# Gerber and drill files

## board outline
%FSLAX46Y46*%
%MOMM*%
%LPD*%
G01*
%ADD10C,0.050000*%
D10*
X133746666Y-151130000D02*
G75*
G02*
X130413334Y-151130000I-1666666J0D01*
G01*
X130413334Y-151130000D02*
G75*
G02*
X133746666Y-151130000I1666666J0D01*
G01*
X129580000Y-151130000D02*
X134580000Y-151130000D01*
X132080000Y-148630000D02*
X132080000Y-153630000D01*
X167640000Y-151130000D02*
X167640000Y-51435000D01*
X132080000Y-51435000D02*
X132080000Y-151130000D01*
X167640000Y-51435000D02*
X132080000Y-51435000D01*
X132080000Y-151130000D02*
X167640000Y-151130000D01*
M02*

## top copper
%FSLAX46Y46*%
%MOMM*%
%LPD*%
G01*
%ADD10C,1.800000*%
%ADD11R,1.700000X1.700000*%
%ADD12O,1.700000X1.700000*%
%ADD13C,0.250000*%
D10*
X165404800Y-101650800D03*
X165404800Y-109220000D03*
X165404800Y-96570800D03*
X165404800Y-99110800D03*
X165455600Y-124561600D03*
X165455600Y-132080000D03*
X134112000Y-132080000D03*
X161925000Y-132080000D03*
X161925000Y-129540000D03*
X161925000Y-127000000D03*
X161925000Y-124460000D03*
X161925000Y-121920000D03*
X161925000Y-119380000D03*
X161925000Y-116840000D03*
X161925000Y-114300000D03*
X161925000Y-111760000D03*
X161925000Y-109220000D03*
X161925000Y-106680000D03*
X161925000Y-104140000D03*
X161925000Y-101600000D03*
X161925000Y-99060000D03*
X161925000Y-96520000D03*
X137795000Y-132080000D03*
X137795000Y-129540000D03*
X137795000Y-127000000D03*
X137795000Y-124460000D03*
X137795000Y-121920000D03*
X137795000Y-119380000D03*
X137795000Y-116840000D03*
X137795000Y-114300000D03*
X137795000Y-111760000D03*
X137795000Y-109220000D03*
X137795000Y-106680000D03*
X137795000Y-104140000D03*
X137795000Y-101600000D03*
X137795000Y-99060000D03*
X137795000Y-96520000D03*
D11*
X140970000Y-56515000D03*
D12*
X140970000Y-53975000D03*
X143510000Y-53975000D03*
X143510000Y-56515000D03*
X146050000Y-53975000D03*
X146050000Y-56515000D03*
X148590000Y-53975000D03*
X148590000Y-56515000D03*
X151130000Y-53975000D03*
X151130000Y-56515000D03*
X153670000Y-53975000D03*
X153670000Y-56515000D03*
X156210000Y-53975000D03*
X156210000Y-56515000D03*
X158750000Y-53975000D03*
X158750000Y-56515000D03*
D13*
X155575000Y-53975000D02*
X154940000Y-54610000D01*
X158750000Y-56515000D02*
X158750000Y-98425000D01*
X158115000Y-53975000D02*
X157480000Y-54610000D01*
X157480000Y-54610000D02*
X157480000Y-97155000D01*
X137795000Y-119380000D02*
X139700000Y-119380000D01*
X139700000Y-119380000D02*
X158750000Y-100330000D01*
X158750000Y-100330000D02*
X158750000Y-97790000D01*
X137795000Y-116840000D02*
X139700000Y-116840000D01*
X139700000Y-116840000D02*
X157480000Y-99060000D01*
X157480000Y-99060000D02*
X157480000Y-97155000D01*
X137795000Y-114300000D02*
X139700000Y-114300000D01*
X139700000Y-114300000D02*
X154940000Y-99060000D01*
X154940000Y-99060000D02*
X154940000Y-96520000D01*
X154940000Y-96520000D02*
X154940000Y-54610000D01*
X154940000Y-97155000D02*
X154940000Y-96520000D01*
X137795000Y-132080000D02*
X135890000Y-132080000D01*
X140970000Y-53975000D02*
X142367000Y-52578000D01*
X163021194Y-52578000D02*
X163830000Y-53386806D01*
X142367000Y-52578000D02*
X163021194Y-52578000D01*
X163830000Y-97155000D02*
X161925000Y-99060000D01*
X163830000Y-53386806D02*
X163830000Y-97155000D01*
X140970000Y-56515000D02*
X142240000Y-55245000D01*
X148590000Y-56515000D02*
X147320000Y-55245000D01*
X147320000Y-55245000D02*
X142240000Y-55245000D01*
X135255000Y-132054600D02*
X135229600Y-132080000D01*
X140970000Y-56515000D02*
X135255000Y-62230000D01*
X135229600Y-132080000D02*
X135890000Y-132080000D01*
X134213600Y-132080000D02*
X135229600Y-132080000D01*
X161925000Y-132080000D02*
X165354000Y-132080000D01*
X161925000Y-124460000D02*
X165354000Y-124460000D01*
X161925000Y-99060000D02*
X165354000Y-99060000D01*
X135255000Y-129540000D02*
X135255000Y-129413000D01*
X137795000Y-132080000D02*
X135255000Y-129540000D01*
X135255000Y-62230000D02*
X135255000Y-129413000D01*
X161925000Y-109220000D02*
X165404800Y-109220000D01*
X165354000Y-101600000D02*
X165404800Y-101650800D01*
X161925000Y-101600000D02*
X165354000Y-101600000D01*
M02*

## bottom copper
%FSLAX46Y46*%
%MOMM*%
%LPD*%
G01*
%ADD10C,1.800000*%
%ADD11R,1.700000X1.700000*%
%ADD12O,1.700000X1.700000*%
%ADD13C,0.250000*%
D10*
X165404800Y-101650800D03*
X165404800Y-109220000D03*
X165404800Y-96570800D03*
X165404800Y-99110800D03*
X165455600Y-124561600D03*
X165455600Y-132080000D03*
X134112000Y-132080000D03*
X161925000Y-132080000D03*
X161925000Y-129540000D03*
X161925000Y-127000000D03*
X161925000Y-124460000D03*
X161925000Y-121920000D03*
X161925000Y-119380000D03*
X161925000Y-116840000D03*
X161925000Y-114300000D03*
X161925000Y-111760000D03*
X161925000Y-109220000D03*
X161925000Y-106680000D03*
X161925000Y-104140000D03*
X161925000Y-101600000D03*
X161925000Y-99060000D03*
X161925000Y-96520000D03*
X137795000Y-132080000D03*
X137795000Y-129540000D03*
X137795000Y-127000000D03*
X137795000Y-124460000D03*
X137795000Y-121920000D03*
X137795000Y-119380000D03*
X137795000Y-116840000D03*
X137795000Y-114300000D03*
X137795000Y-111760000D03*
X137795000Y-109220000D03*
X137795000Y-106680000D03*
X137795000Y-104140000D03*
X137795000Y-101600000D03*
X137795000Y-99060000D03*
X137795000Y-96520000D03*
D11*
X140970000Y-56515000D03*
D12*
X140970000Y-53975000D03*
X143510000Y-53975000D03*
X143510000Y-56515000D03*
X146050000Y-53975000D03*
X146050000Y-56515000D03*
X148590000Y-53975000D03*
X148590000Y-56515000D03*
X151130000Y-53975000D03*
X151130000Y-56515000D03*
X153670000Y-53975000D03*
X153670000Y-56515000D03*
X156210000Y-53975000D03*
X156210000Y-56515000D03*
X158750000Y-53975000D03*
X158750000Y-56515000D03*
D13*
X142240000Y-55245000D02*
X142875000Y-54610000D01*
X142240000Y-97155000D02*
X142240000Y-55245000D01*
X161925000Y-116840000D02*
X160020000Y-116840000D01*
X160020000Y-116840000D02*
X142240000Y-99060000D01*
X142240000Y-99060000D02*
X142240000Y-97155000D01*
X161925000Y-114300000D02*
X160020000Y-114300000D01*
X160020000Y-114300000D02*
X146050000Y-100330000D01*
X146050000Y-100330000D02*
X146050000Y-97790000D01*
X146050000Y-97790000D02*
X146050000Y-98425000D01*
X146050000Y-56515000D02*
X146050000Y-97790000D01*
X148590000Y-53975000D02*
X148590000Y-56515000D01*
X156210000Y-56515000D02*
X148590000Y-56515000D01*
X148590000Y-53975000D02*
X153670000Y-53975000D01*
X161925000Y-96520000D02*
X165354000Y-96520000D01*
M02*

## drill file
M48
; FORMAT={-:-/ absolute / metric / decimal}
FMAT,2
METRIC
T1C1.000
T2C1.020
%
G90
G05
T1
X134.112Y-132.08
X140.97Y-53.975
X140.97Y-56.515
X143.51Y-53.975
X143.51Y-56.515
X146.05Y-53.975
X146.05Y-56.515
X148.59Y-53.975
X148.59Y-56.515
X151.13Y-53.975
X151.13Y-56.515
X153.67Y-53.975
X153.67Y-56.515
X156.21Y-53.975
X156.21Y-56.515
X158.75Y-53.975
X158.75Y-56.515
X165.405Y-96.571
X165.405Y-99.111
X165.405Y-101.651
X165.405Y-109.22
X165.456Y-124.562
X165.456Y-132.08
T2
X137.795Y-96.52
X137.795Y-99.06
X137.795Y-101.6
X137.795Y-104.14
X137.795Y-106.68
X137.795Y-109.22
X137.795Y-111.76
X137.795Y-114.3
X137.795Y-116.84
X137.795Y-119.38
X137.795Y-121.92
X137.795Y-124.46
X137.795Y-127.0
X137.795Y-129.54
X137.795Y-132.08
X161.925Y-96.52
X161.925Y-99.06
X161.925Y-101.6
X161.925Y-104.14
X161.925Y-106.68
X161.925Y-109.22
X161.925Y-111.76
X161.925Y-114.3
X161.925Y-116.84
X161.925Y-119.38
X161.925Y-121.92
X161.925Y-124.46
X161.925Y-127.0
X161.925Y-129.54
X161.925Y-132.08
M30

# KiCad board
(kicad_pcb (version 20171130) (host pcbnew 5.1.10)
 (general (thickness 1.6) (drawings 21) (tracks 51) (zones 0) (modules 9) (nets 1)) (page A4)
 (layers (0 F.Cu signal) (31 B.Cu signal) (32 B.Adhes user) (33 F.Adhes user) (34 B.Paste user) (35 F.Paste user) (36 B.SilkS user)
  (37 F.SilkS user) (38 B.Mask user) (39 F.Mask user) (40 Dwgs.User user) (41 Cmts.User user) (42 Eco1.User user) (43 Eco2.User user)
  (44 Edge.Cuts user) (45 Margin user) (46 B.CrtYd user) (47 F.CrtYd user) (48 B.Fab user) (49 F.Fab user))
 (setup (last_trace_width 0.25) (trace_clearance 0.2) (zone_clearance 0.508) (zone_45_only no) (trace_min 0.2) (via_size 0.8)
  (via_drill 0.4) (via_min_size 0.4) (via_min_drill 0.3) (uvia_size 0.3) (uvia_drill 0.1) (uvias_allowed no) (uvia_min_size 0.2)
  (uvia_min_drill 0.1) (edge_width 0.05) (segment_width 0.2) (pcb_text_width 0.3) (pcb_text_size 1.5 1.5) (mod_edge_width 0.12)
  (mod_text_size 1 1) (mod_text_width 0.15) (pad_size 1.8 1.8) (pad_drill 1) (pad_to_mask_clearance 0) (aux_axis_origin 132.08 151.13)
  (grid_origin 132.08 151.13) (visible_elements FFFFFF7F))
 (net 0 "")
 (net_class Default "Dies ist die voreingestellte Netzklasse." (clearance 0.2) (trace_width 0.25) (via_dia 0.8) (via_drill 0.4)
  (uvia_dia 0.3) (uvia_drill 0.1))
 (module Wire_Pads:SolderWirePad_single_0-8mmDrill (layer F.Cu) (at 165.4048 101.6508)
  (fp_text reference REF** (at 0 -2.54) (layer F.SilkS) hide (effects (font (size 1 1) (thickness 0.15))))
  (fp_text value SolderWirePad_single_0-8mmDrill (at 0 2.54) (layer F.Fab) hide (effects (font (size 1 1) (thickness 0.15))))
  (pad 1 thru_hole circle (at 0 0) (size 1.8 1.8) (drill 1) (layers *.Cu *.Mask)))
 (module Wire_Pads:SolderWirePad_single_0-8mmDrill (layer F.Cu) (at 165.4048 109.22)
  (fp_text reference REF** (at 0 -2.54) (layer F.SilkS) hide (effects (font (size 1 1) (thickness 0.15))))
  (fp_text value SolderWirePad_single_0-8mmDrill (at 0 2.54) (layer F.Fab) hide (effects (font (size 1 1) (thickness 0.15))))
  (pad 1 thru_hole circle (at 0 0) (size 1.8 1.8) (drill 1) (layers *.Cu *.Mask)))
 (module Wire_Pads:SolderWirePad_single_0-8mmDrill (layer F.Cu) (at 165.4048 96.5708)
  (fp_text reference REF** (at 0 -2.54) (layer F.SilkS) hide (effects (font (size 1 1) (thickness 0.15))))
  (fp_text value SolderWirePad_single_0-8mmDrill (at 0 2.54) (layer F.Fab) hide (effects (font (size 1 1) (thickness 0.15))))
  (pad 1 thru_hole circle (at 0 0) (size 1.8 1.8) (drill 1) (layers *.Cu *.Mask)))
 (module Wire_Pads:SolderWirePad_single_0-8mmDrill (layer F.Cu) (at 165.4048 99.1108)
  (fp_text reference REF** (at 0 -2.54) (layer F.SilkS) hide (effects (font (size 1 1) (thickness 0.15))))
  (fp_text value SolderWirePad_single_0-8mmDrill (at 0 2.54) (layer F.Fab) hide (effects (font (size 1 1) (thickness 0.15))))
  (pad 1 thru_hole circle (at 0 0) (size 1.8 1.8) (drill 1) (layers *.Cu *.Mask)))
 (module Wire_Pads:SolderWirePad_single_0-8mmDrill (layer F.Cu) (at 165.4556 124.5616)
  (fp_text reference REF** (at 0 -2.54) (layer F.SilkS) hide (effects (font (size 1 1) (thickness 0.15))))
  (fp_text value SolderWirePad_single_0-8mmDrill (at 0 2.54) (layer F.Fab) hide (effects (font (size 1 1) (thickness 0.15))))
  (pad 1 thru_hole circle (at 0 0) (size 1.8 1.8) (drill 1) (layers *.Cu *.Mask)))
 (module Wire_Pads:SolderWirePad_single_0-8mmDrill (layer F.Cu) (at 165.4556 132.08)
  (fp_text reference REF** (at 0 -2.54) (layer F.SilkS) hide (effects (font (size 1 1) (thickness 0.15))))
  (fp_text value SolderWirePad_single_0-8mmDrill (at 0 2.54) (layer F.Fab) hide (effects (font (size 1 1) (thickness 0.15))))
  (pad 1 thru_hole circle (at 0 0) (size 1.8 1.8) (drill 1) (layers *.Cu *.Mask)))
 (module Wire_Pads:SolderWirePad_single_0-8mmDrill (layer F.Cu) (at 134.112 132.08)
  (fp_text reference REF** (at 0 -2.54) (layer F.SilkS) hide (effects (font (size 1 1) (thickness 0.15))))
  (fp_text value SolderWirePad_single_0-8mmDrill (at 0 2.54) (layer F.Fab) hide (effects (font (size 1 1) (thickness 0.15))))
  (pad 1 thru_hole circle (at 0 0) (size 1.8 1.8) (drill 1) (layers *.Cu *.Mask)))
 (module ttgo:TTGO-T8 (layer F.Cu) (at 137.795 96.52)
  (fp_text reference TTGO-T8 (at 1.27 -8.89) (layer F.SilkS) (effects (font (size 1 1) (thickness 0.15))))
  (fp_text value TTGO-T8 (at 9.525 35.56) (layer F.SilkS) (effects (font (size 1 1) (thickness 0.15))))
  (pad 5V thru_hole circle (at 24.13 35.56) (size 1.8 1.8) (drill 1.02) (layers *.Cu *.Mask))
  (pad 4 thru_hole circle (at 24.13 33.02) (size 1.8 1.8) (drill 1.02) (layers *.Cu *.Mask))
  (pad 0 thru_hole circle (at 24.13 30.48) (size 1.8 1.8) (drill 1.02) (layers *.Cu *.Mask))
  (pad GND thru_hole circle (at 24.13 27.94) (size 1.8 1.8) (drill 1.02) (layers *.Cu *.Mask))
  (pad 2 thru_hole circle (at 24.13 25.4) (size 1.8 1.8) (drill 1.02) (layers *.Cu *.Mask))
  (pad 5 thru_hole circle (at 24.13 22.86) (size 1.8 1.8) (drill 1.02) (layers *.Cu *.Mask))
  (pad 18 thru_hole circle (at 24.13 20.32) (size 1.8 1.8) (drill 1.02) (layers *.Cu *.Mask))
  (pad 23 thru_hole circle (at 24.13 17.78) (size 1.8 1.8) (drill 1.02) (layers *.Cu *.Mask))
  (pad 19 thru_hole circle (at 24.13 15.24) (size 1.8 1.8) (drill 1.02) (layers *.Cu *.Mask))
  (pad 22 thru_hole circle (at 24.13 12.7) (size 1.8 1.8) (drill 1.02) (layers *.Cu *.Mask))
  (pad RXD thru_hole circle (at 24.13 10.16) (size 1.8 1.8) (drill 1.02) (layers *.Cu *.Mask))
  (pad TXD thru_hole circle (at 24.13 7.62) (size 1.8 1.8) (drill 1.02) (layers *.Cu *.Mask))
  (pad 21 thru_hole circle (at 24.13 5.08) (size 1.8 1.8) (drill 1.02) (layers *.Cu *.Mask))
  (pad 3-3 thru_hole circle (at 24.13 2.54) (size 1.8 1.8) (drill 1.02) (layers *.Cu *.Mask))
  (pad GND thru_hole circle (at 24.13 0) (size 1.8 1.8) (drill 1.02) (layers *.Cu *.Mask))
  (pad GND thru_hole circle (at 0 35.56) (size 1.8 1.8) (drill 1.02) (layers *.Cu *.Mask))
  (pad 15 thru_hole circle (at 0 33.02) (size 1.8 1.8) (drill 1.02) (layers *.Cu *.Mask))
  (pad 13 thru_hole circle (at 0 30.48) (size 1.8 1.8) (drill 1.02) (layers *.Cu *.Mask))
  (pad 12 thru_hole circle (at 0 27.94) (size 1.8 1.8) (drill 1.02) (layers *.Cu *.Mask))
  (pad 14 thru_hole circle (at 0 25.4) (size 1.8 1.8) (drill 1.02) (layers *.Cu *.Mask))
  (pad 27 thru_hole circle (at 0 22.86) (size 1.8 1.8) (drill 1.02) (layers *.Cu *.Mask))
  (pad 26 thru_hole circle (at 0 20.32) (size 1.8 1.8) (drill 1.02) (layers *.Cu *.Mask))
  (pad 25 thru_hole circle (at 0 17.78) (size 1.8 1.8) (drill 1.02) (layers *.Cu *.Mask))
  (pad 33 thru_hole circle (at 0 15.24) (size 1.8 1.8) (drill 1.02) (layers *.Cu *.Mask))
  (pad 32 thru_hole circle (at 0 12.7) (size 1.8 1.8) (drill 1.02) (layers *.Cu *.Mask))
  (pad 35 thru_hole circle (at 0 10.16) (size 1.8 1.8) (drill 1.02) (layers *.Cu *.Mask))
  (pad 34 thru_hole circle (at 0 7.62) (size 1.8 1.8) (drill 1.02) (layers *.Cu *.Mask))
  (pad RST thru_hole circle (at 0 5.08) (size 1.8 1.8) (drill 1.02) (layers *.Cu *.Mask))
  (pad VN thru_hole circle (at 0 2.54) (size 1.8 1.8) (drill 1.02) (layers *.Cu *.Mask))
  (pad VP thru_hole circle (at 0 0) (size 1.8 1.8) (drill 1.02) (layers *.Cu *.Mask)))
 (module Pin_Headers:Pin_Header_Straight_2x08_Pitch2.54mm (layer B.Cu) (at 140.97 53.975 270)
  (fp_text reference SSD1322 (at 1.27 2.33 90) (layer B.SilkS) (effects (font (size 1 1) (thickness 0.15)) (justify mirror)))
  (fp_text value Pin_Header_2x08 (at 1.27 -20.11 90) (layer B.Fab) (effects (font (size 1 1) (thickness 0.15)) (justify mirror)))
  (pad 1 thru_hole rect (at 2.54 0 270) (size 1.7 1.7) (drill 1) (layers *.Cu *.Mask))
  (pad 2 thru_hole oval (at 0 0 270) (size 1.7 1.7) (drill 1) (layers *.Cu *.Mask))
  (pad 4 thru_hole oval (at 0 -2.54 270) (size 1.7 1.7) (drill 1) (layers *.Cu *.Mask))
  (pad 3 thru_hole oval (at 2.54 -2.54 270) (size 1.7 1.7) (drill 1) (layers *.Cu *.Mask))
  (pad 6 thru_hole oval (at 0 -5.08 270) (size 1.7 1.7) (drill 1) (layers *.Cu *.Mask))
  (pad 5 thru_hole oval (at 2.54 -5.08 270) (size 1.7 1.7) (drill 1) (layers *.Cu *.Mask))
  (pad 8 thru_hole oval (at 0 -7.62 270) (size 1.7 1.7) (drill 1) (layers *.Cu *.Mask))
  (pad 7 thru_hole oval (at 2.54 -7.62 270) (size 1.7 1.7) (drill 1) (layers *.Cu *.Mask))
  (pad 10 thru_hole oval (at 0 -10.16 270) (size 1.7 1.7) (drill 1) (layers *.Cu *.Mask))
  (pad 9 thru_hole oval (at 2.54 -10.16 270) (size 1.7 1.7) (drill 1) (layers *.Cu *.Mask))
  (pad 12 thru_hole oval (at 0 -12.7 270) (size 1.7 1.7) (drill 1) (layers *.Cu *.Mask))
  (pad 11 thru_hole oval (at 2.54 -12.7 270) (size 1.7 1.7) (drill 1) (layers *.Cu *.Mask))
  (pad 14 thru_hole oval (at 0 -15.24 270) (size 1.7 1.7) (drill 1) (layers *.Cu *.Mask))
  (pad 13 thru_hole oval (at 2.54 -15.24 270) (size 1.7 1.7) (drill 1) (layers *.Cu *.Mask))
  (pad 16 thru_hole oval (at 0 -17.78 270) (size 1.7 1.7) (drill 1) (layers *.Cu *.Mask))
  (pad 15 thru_hole oval (at 2.54 -17.78 270) (size 1.7 1.7) (drill 1) (layers *.Cu *.Mask)))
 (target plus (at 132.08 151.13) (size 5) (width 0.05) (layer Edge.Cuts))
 (gr_line (start 167.64 151.13) (end 167.64 51.435) (layer Edge.Cuts) (width 0.05))
 (gr_line (start 132.08 51.435) (end 132.08 151.13) (layer Edge.Cuts) (width 0.05))
 (gr_line (start 167.64 51.435) (end 132.08 51.435) (layer Edge.Cuts) (width 0.05))
 (gr_line (start 132.08 151.13) (end 167.64 151.13) (layer Edge.Cuts) (width 0.05))
 (segment (start 142.24 55.245) (end 142.875 54.61) (width 0.25) (layer B.Cu) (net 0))
 (segment (start 142.24 97.155) (end 142.24 55.245) (width 0.25) (layer B.Cu) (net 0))
 (segment (start 155.575 53.975) (end 154.94 54.61) (width 0.25) (layer F.Cu) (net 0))
 (segment (start 158.75 56.515) (end 158.75 98.425) (width 0.25) (layer F.Cu) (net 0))
 (segment (start 158.115 53.975) (end 157.48 54.61) (width 0.25) (layer F.Cu) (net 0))
 (segment (start 157.48 54.61) (end 157.48 97.155) (width 0.25) (layer F.Cu) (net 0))
 (segment (start 161.925 116.84) (end 160.02 116.84) (width 0.25) (layer B.Cu) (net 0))
 (segment (start 160.02 116.84) (end 142.24 99.06) (width 0.25) (layer B.Cu) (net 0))
 (segment (start 142.24 99.06) (end 142.24 97.155) (width 0.25) (layer B.Cu) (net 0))
 (segment (start 161.925 114.3) (end 160.02 114.3) (width 0.25) (layer B.Cu) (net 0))
 (segment (start 160.02 114.3) (end 146.05 100.33) (width 0.25) (layer B.Cu) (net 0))
 (segment (start 146.05 100.33) (end 146.05 97.79) (width 0.25) (layer B.Cu) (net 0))
 (segment (start 146.05 97.79) (end 146.05 98.425) (width 0.25) (layer B.Cu) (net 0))
 (segment (start 146.05 56.515) (end 146.05 97.79) (width 0.25) (layer B.Cu) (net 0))
 (segment (start 137.795 119.38) (end 139.7 119.38) (width 0.25) (layer F.Cu) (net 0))
 (segment (start 139.7 119.38) (end 158.75 100.33) (width 0.25) (layer F.Cu) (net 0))
 (segment (start 158.75 100.33) (end 158.75 97.79) (width 0.25) (layer F.Cu) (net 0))
 (segment (start 137.795 116.84) (end 139.7 116.84) (width 0.25) (layer F.Cu) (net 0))
 (segment (start 139.7 116.84) (end 157.48 99.06) (width 0.25) (layer F.Cu) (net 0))
 (segment (start 157.48 99.06) (end 157.48 97.155) (width 0.25) (layer F.Cu) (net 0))
 (segment (start 137.795 114.3) (end 139.7 114.3) (width 0.25) (layer F.Cu) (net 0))
 (segment (start 139.7 114.3) (end 154.94 99.06) (width 0.25) (layer F.Cu) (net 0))
 (segment (start 154.94 99.06) (end 154.94 96.52) (width 0.25) (layer F.Cu) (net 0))
 (segment (start 154.94 96.52) (end 154.94 54.61) (width 0.25) (layer F.Cu) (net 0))
 (segment (start 154.94 97.155) (end 154.94 96.52) (width 0.25) (layer F.Cu) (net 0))
 (segment (start 137.795 132.08) (end 135.89 132.08) (width 0.25) (layer F.Cu) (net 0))
 (segment (start 140.97 53.975) (end 142.367 52.578) (width 0.25) (layer F.Cu) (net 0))
 (segment (start 163.021194 52.578) (end 163.83 53.386806) (width 0.25) (layer F.Cu) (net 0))
 (segment (start 142.367 52.578) (end 163.021194 52.578) (width 0.25) (layer F.Cu) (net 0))
 (segment (start 163.83 97.155) (end 161.925 99.06) (width 0.25) (layer F.Cu) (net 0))
 (segment (start 163.83 53.386806) (end 163.83 97.155) (width 0.25) (layer F.Cu) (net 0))
 (segment (start 148.59 53.975) (end 148.59 56.515) (width 0.25) (layer B.Cu) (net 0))
 (segment (start 156.21 56.515) (end 148.59 56.515) (width 0.25) (layer B.Cu) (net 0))
 (segment (start 148.59 53.975) (end 153.67 53.975) (width 0.25) (layer B.Cu) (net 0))
 (segment (start 140.97 56.515) (end 142.24 55.245) (width 0.25) (layer F.Cu) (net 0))
 (segment (start 148.59 56.515) (end 147.32 55.245) (width 0.25) (layer F.Cu) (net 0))
 (segment (start 147.32 55.245) (end 142.24 55.245) (width 0.25) (layer F.Cu) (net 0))
 (segment (start 135.255 132.0546) (end 135.2296 132.08) (width 0.25) (layer F.Cu) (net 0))
 (segment (start 140.97 56.515) (end 135.255 62.23) (width 0.25) (layer F.Cu) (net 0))
 (segment (start 135.2296 132.08) (end 135.89 132.08) (width 0.25) (layer F.Cu) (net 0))
 (segment (start 134.2136 132.08) (end 135.2296 132.08) (width 0.25) (layer F.Cu) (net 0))
 (segment (start 161.925 132.08) (end 165.354 132.08) (width 0.25) (layer F.Cu) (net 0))
 (segment (start 161.925 124.46) (end 165.354 124.46) (width 0.25) (layer F.Cu) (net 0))
 (segment (start 161.925 99.06) (end 165.354 99.06) (width 0.25) (layer F.Cu) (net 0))
 (segment (start 161.925 96.52) (end 165.354 96.52) (width 0.25) (layer B.Cu) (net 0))
 (segment (start 135.255 129.54) (end 135.255 129.413) (width 0.25) (layer F.Cu) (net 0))
 (segment (start 137.795 132.08) (end 135.255 129.54) (width 0.25) (layer F.Cu) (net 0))
 (segment (start 135.255 62.23) (end 135.255 129.413) (width 0.25) (layer F.Cu) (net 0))
 (segment (start 161.925 109.22) (end 165.4048 109.22) (width 0.25) (layer F.Cu) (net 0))
 (segment (start 165.354 101.6) (end 165.4048 101.6508) (width 0.25) (layer F.Cu) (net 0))
 (segment (start 161.925 101.6) (end 165.354 101.6) (width 0.25) (layer F.Cu) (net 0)))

